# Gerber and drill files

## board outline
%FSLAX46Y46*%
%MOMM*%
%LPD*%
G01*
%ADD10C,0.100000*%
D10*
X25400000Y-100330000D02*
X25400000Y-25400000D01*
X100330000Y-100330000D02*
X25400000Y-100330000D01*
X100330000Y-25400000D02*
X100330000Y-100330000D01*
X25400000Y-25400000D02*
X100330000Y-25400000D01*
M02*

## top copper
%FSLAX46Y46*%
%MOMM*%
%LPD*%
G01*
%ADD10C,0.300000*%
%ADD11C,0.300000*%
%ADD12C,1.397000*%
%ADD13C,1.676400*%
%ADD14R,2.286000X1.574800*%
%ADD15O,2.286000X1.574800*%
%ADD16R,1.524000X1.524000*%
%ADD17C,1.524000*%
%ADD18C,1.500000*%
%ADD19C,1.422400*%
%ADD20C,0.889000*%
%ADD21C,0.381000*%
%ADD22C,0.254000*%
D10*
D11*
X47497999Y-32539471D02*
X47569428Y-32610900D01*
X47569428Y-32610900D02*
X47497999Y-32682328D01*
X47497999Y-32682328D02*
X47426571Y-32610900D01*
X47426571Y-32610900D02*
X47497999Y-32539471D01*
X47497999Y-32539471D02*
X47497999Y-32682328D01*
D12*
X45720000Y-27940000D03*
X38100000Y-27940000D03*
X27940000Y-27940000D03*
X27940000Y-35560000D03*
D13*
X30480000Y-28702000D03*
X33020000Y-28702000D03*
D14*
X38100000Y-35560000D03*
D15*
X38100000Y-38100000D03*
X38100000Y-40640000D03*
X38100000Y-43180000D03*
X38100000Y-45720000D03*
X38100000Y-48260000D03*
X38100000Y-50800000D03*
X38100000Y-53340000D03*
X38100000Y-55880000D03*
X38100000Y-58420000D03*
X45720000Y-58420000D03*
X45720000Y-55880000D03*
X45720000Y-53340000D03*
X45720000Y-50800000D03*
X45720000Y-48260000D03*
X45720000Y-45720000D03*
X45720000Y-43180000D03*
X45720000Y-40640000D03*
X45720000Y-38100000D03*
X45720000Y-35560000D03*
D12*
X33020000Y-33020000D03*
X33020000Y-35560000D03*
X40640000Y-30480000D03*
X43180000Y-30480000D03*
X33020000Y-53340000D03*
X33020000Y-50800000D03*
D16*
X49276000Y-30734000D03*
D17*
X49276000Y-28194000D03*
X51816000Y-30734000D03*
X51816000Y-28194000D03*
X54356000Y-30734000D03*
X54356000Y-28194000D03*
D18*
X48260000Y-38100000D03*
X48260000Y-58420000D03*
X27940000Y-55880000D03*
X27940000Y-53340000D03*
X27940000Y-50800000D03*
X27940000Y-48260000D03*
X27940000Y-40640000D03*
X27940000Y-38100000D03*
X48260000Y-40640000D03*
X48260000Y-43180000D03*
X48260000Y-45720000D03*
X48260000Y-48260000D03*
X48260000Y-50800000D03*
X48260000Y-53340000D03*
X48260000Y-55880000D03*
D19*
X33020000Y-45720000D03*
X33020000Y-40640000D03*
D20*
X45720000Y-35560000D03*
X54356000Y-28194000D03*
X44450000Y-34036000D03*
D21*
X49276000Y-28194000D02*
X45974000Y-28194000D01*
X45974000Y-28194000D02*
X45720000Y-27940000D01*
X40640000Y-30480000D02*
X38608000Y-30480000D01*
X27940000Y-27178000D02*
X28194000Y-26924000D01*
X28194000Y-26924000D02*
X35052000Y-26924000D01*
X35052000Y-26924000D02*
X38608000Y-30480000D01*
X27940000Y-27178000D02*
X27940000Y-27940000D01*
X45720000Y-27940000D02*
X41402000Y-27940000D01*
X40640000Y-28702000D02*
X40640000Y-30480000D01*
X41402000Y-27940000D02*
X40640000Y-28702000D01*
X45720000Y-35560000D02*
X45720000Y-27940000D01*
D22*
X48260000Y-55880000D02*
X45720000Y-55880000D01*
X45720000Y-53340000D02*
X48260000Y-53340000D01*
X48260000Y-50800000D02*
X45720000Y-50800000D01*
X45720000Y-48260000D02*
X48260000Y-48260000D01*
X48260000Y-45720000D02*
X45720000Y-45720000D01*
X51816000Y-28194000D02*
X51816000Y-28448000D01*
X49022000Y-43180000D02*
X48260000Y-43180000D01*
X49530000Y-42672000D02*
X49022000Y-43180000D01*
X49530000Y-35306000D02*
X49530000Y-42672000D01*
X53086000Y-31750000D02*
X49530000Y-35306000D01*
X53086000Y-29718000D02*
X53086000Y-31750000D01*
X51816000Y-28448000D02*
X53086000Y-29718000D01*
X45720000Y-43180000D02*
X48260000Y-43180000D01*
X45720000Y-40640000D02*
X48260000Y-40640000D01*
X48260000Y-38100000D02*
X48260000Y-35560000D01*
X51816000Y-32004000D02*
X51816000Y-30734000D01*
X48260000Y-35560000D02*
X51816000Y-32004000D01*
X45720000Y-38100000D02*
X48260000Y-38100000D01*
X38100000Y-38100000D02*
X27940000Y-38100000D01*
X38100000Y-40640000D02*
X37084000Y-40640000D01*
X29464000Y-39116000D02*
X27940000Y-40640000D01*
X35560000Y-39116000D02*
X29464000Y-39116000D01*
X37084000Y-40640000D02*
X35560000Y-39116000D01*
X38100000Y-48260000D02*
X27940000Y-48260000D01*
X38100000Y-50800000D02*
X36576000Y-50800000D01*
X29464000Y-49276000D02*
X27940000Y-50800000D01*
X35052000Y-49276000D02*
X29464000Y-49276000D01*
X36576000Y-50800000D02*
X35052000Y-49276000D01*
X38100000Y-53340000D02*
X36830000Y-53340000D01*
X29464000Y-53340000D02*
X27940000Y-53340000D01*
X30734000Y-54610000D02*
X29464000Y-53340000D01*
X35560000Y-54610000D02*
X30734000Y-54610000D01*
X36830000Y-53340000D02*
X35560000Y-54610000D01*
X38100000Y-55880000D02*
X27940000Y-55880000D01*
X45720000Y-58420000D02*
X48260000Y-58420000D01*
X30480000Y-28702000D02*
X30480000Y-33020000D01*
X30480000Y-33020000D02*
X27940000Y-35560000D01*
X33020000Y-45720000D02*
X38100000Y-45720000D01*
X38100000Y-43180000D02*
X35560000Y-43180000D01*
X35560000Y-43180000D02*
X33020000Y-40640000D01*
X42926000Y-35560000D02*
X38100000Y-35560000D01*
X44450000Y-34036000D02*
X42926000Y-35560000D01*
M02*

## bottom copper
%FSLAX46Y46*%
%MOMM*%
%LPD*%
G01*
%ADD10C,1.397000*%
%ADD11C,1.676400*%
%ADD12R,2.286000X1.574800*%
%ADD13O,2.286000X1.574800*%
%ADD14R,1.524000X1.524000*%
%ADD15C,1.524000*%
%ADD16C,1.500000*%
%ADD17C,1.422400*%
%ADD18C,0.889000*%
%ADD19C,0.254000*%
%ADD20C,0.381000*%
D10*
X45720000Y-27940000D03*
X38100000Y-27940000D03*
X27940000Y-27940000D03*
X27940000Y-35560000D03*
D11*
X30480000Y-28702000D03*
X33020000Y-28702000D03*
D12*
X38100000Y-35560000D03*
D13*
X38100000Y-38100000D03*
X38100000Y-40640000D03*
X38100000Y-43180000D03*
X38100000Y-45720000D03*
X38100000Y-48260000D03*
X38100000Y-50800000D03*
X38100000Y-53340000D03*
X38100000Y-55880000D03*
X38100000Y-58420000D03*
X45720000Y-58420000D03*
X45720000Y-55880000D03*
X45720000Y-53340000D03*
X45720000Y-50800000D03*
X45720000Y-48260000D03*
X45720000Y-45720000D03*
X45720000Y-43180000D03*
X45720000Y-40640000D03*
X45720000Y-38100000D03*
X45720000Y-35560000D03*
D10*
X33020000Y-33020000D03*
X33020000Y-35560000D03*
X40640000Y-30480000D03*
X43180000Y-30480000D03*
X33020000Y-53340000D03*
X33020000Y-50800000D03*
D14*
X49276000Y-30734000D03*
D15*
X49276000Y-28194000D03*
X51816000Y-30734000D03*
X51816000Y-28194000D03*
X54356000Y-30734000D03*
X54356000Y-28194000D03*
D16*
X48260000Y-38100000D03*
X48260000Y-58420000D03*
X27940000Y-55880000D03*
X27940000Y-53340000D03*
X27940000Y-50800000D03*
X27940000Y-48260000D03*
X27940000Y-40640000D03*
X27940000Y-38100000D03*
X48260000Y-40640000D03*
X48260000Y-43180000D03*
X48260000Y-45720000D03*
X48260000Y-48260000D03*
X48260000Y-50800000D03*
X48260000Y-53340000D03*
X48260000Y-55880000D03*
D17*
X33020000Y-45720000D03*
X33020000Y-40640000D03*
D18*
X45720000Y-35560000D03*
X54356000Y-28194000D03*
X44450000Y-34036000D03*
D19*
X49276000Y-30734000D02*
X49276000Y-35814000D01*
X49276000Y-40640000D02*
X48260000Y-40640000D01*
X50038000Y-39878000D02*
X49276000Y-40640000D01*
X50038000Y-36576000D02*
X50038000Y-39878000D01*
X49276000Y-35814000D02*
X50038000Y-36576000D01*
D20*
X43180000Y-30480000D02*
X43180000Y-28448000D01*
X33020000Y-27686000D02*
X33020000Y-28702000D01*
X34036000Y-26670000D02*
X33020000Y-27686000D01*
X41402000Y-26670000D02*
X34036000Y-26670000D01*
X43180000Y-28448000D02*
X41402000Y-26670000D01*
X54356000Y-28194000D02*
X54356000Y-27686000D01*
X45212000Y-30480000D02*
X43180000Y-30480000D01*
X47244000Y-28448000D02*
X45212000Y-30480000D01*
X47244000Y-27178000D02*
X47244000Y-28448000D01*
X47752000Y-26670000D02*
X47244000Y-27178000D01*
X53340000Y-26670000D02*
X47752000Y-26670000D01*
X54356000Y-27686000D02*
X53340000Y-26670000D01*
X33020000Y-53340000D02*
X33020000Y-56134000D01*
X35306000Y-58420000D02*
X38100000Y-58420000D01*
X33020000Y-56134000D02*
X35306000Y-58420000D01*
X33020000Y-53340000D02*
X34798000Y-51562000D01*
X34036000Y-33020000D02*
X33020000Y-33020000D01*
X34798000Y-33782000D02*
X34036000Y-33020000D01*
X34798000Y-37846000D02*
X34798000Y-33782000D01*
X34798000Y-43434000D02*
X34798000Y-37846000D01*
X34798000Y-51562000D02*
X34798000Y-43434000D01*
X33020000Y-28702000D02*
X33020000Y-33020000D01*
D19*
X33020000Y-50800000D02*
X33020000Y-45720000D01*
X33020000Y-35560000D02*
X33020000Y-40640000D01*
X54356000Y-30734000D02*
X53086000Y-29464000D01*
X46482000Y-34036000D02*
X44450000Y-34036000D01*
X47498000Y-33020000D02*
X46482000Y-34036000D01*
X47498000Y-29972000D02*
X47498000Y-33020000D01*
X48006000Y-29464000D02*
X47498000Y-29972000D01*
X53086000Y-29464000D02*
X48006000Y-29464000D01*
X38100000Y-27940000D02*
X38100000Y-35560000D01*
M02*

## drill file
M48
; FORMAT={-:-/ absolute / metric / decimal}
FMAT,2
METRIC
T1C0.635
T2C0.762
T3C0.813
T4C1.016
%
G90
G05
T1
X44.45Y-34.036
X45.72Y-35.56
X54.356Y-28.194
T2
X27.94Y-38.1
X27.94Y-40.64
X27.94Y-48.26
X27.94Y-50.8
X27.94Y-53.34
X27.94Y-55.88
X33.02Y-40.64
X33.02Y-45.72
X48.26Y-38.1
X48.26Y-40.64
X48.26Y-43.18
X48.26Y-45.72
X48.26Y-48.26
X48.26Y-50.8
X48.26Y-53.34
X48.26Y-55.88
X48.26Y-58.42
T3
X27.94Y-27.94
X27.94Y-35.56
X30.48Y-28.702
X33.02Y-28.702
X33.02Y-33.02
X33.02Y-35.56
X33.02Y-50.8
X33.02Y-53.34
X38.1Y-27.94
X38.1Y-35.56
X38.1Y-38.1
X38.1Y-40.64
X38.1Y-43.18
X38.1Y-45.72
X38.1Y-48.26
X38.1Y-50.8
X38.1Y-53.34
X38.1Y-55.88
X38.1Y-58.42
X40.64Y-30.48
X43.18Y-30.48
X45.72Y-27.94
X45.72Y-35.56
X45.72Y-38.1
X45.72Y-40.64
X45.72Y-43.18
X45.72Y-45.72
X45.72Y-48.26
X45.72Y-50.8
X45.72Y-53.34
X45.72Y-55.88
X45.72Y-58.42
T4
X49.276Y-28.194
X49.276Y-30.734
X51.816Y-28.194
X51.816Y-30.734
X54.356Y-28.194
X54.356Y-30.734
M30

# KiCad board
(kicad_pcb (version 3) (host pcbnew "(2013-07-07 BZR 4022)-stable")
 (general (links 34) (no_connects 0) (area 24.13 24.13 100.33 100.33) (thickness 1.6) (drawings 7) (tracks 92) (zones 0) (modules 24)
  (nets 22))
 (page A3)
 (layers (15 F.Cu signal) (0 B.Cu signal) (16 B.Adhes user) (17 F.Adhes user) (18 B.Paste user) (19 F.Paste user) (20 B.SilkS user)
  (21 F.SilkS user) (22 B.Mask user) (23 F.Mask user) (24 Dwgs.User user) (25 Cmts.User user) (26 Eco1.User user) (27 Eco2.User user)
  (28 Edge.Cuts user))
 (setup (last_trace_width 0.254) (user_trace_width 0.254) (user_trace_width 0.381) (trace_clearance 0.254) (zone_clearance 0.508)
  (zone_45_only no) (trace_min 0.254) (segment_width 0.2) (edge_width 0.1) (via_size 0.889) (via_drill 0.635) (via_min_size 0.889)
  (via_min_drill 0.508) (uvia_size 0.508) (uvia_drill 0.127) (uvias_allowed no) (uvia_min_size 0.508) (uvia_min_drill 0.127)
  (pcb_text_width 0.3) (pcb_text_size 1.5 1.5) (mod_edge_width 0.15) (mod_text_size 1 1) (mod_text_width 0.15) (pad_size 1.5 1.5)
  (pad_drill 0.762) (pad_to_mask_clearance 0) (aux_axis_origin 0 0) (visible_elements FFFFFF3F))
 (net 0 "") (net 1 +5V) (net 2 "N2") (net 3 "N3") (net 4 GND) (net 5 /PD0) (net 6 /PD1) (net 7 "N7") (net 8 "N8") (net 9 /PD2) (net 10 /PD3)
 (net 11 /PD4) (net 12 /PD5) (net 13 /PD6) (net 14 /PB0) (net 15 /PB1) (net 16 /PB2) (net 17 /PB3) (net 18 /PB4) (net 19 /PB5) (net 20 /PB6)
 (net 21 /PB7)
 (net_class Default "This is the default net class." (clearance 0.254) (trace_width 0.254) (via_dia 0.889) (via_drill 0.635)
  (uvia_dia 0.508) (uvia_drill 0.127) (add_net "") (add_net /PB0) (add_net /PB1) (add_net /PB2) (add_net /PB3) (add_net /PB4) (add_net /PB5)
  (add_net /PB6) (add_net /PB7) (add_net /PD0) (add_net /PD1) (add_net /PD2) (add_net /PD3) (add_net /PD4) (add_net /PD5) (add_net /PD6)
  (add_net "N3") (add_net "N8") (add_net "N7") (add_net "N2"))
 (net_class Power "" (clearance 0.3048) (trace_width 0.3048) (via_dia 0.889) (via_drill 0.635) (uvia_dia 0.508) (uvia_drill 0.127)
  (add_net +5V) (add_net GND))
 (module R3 (layer F.Cu) (at 41.91 27.94 180) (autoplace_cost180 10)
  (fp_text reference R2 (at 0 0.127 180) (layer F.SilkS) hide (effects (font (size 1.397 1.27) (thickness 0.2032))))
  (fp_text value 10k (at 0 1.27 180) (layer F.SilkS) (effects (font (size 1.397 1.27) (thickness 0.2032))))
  (pad 1 thru_hole circle (at -3.81 0 180) (size 1.397 1.397) (drill 0.8128) (layers *.Cu *.Mask F.SilkS) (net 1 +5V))
  (pad 2 thru_hole circle (at 3.81 0 180) (size 1.397 1.397) (drill 0.8128) (layers *.Cu *.Mask F.SilkS) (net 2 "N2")))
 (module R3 (layer F.Cu) (at 27.94 31.75 270) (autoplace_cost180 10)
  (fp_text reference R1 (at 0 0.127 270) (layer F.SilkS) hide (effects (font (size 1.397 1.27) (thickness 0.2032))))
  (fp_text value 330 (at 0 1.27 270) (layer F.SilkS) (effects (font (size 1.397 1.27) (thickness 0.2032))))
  (pad 1 thru_hole circle (at -3.81 0 270) (size 1.397 1.397) (drill 0.8128) (layers *.Cu *.Mask F.SilkS) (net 1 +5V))
  (pad 2 thru_hole circle (at 3.81 0 270) (size 1.397 1.397) (drill 0.8128) (layers *.Cu *.Mask F.SilkS) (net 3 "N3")))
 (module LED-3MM (layer F.Cu) (at 31.75 28.702)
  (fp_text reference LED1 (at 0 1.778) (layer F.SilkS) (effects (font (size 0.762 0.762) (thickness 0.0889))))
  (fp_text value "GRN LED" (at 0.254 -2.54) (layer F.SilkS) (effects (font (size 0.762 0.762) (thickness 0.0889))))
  (pad 1 thru_hole circle (at -1.27 0) (size 1.6764 1.6764) (drill 0.8128) (layers *.Cu *.Mask F.SilkS) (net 3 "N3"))
  (pad 2 thru_hole circle (at 1.27 0) (size 1.6764 1.6764) (drill 0.8128) (layers *.Cu *.Mask F.SilkS) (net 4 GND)))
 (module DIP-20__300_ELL (layer F.Cu) (at 41.91 46.99 270)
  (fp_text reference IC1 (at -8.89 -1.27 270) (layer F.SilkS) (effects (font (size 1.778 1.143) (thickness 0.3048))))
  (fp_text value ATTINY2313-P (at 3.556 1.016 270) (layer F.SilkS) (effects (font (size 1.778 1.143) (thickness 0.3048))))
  (pad 1 thru_hole rect (at -11.43 3.81 270) (size 1.5748 2.286) (drill 0.8128) (layers *.Cu *.Mask F.SilkS) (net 2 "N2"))
  (pad 2 thru_hole oval (at -8.89 3.81 270) (size 1.5748 2.286) (drill 0.8128) (layers *.Cu *.Mask F.SilkS) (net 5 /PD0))
  (pad 3 thru_hole oval (at -6.35 3.81 270) (size 1.5748 2.286) (drill 0.8128) (layers *.Cu *.Mask F.SilkS) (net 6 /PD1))
  (pad 4 thru_hole oval (at -3.81 3.81 270) (size 1.5748 2.286) (drill 0.8128) (layers *.Cu *.Mask F.SilkS) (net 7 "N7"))
  (pad 5 thru_hole oval (at -1.27 3.81 270) (size 1.5748 2.286) (drill 0.8128) (layers *.Cu *.Mask F.SilkS) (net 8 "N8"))
  (pad 6 thru_hole oval (at 1.27 3.81 270) (size 1.5748 2.286) (drill 0.8128) (layers *.Cu *.Mask F.SilkS) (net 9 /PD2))
  (pad 7 thru_hole oval (at 3.81 3.81 270) (size 1.5748 2.286) (drill 0.8128) (layers *.Cu *.Mask F.SilkS) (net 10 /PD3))
  (pad 8 thru_hole oval (at 6.35 3.81 270) (size 1.5748 2.286) (drill 0.8128) (layers *.Cu *.Mask F.SilkS) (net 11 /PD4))
  (pad 9 thru_hole oval (at 8.89 3.81 270) (size 1.5748 2.286) (drill 0.8128) (layers *.Cu *.Mask F.SilkS) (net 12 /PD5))
  (pad 10 thru_hole oval (at 11.43 3.81 270) (size 1.5748 2.286) (drill 0.8128) (layers *.Cu *.Mask F.SilkS) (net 4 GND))
  (pad 11 thru_hole oval (at 11.43 -3.81 270) (size 1.5748 2.286) (drill 0.8128) (layers *.Cu *.Mask F.SilkS) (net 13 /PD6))
  (pad 12 thru_hole oval (at 8.89 -3.81 270) (size 1.5748 2.286) (drill 0.8128) (layers *.Cu *.Mask F.SilkS) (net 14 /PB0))
  (pad 13 thru_hole oval (at 6.35 -3.81 270) (size 1.5748 2.286) (drill 0.8128) (layers *.Cu *.Mask F.SilkS) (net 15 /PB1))
  (pad 14 thru_hole oval (at 3.81 -3.81 270) (size 1.5748 2.286) (drill 0.8128) (layers *.Cu *.Mask F.SilkS) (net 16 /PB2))
  (pad 15 thru_hole oval (at 1.27 -3.81 270) (size 1.5748 2.286) (drill 0.8128) (layers *.Cu *.Mask F.SilkS) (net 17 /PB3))
  (pad 16 thru_hole oval (at -1.27 -3.81 270) (size 1.5748 2.286) (drill 0.8128) (layers *.Cu *.Mask F.SilkS) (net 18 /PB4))
  (pad 17 thru_hole oval (at -3.81 -3.81 270) (size 1.5748 2.286) (drill 0.8128) (layers *.Cu *.Mask F.SilkS) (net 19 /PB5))
  (pad 18 thru_hole oval (at -6.35 -3.81 270) (size 1.5748 2.286) (drill 0.8128) (layers *.Cu *.Mask F.SilkS) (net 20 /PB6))
  (pad 19 thru_hole oval (at -8.89 -3.81 270) (size 1.5748 2.286) (drill 0.8128) (layers *.Cu *.Mask F.SilkS) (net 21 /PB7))
  (pad 20 thru_hole oval (at -11.43 -3.81 270) (size 1.5748 2.286) (drill 0.8128) (layers *.Cu *.Mask F.SilkS) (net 1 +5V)))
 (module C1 (layer F.Cu) (at 33.02 34.29 270)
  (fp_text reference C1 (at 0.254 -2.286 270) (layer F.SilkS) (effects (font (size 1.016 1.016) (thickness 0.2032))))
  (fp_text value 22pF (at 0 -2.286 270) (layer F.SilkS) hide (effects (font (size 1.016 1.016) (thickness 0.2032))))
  (pad 1 thru_hole circle (at -1.27 0 270) (size 1.397 1.397) (drill 0.8128) (layers *.Cu *.Mask F.SilkS) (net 4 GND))
  (pad 2 thru_hole circle (at 1.27 0 270) (size 1.397 1.397) (drill 0.8128) (layers *.Cu *.Mask F.SilkS) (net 7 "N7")))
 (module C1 (layer F.Cu) (at 41.91 30.48)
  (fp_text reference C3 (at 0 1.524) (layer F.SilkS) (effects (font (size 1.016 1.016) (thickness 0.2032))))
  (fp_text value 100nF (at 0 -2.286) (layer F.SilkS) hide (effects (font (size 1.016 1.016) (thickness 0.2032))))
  (pad 1 thru_hole circle (at -1.27 0) (size 1.397 1.397) (drill 0.8128) (layers *.Cu *.Mask F.SilkS) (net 1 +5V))
  (pad 2 thru_hole circle (at 1.27 0) (size 1.397 1.397) (drill 0.8128) (layers *.Cu *.Mask F.SilkS) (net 4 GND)))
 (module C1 (layer F.Cu) (at 33.02 52.07 90)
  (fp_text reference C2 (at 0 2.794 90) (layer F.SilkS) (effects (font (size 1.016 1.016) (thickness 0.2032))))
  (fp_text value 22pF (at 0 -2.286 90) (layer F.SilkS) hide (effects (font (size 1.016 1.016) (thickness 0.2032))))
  (pad 1 thru_hole circle (at -1.27 0 90) (size 1.397 1.397) (drill 0.8128) (layers *.Cu *.Mask F.SilkS) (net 4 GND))
  (pad 2 thru_hole circle (at 1.27 0 90) (size 1.397 1.397) (drill 0.8128) (layers *.Cu *.Mask F.SilkS) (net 8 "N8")))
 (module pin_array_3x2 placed (layer F.Cu) (at 51.816 29.464)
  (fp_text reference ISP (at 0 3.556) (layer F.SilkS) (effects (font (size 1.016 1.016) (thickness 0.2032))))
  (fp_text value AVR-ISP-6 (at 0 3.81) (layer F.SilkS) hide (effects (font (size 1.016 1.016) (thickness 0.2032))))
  (pad 1 thru_hole rect (at -2.54 1.27) (size 1.524 1.524) (drill 1.016) (layers *.Cu *.Mask F.SilkS) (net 20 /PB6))
  (pad 2 thru_hole circle (at -2.54 -1.27) (size 1.524 1.524) (drill 1.016) (layers *.Cu *.Mask F.SilkS) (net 1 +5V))
  (pad 3 thru_hole circle (at 0 1.27) (size 1.524 1.524) (drill 1.016) (layers *.Cu *.Mask F.SilkS) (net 21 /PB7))
  (pad 4 thru_hole circle (at 0 -1.27) (size 1.524 1.524) (drill 1.016) (layers *.Cu *.Mask F.SilkS) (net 19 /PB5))
  (pad 5 thru_hole circle (at 2.54 1.27) (size 1.524 1.524) (drill 1.016) (layers *.Cu *.Mask F.SilkS) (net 2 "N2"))
  (pad 6 thru_hole circle (at 2.54 -1.27) (size 1.524 1.524) (drill 1.016) (layers *.Cu *.Mask F.SilkS) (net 4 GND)))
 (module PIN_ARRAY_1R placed (layer F.Cu) (at 48.26 38.1)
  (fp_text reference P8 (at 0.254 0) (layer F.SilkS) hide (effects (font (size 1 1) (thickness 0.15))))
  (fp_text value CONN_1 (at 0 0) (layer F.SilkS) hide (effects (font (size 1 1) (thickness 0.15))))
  (pad 1 thru_hole circle (at 0 0) (size 1.5 1.5) (drill 0.762) (layers *.Cu *.Mask F.SilkS) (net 21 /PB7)))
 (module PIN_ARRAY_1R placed (layer F.Cu) (at 48.26 58.42)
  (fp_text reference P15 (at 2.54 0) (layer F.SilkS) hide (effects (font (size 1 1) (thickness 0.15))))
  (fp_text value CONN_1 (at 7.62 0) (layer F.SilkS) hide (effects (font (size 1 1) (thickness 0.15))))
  (pad 1 thru_hole circle (at 0 0) (size 1.5 1.5) (drill 0.762) (layers *.Cu *.Mask F.SilkS) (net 13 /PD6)))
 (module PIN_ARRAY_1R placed (layer F.Cu) (at 27.94 55.88)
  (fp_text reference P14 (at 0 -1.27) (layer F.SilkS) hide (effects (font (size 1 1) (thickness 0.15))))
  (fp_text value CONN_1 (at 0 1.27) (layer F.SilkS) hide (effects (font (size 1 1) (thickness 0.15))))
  (pad 1 thru_hole circle (at 0 0) (size 1.5 1.5) (drill 0.762) (layers *.Cu *.Mask F.SilkS) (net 12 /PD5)))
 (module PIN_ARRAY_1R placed (layer F.Cu) (at 27.94 53.34)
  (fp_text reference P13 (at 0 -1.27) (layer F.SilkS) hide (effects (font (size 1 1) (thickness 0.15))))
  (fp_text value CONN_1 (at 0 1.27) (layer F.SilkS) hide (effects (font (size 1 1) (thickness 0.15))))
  (pad 1 thru_hole circle (at 0 0) (size 1.5 1.5) (drill 0.762) (layers *.Cu *.Mask F.SilkS) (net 11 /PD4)))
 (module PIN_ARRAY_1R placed (layer F.Cu) (at 27.94 50.8)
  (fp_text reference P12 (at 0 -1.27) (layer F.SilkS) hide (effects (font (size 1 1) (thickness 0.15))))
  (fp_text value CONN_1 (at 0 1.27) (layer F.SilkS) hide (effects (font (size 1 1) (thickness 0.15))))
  (pad 1 thru_hole circle (at 0 0) (size 1.5 1.5) (drill 0.762) (layers *.Cu *.Mask F.SilkS) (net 10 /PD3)))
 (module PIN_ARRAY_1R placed (layer F.Cu) (at 27.94 48.26)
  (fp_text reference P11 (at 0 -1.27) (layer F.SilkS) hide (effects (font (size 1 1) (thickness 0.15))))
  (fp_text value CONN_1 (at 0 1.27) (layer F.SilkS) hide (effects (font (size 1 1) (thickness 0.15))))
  (pad 1 thru_hole circle (at 0 0) (size 1.5 1.5) (drill 0.762) (layers *.Cu *.Mask F.SilkS) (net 9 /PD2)))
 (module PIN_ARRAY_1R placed (layer F.Cu) (at 27.94 40.64)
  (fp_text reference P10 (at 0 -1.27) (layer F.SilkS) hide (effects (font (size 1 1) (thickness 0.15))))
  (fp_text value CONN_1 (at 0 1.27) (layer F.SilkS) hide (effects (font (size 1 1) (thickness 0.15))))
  (pad 1 thru_hole circle (at 0 0) (size 1.5 1.5) (drill 0.762) (layers *.Cu *.Mask F.SilkS) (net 6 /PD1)))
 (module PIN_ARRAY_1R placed (layer F.Cu) (at 27.94 38.1)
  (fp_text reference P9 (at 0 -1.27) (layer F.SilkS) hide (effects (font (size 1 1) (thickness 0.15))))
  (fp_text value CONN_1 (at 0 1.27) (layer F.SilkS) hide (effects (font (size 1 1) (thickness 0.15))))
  (pad 1 thru_hole circle (at 0 0) (size 1.5 1.5) (drill 0.762) (layers *.Cu *.Mask F.SilkS) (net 5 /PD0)))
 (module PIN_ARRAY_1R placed (layer F.Cu) (at 48.26 40.64)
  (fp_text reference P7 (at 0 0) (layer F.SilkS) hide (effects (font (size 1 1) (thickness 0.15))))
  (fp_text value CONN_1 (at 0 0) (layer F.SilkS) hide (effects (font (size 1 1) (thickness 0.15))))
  (pad 1 thru_hole circle (at 0 0) (size 1.5 1.5) (drill 0.762) (layers *.Cu *.Mask F.SilkS) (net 20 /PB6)))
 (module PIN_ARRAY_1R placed (layer F.Cu) (at 48.26 43.18)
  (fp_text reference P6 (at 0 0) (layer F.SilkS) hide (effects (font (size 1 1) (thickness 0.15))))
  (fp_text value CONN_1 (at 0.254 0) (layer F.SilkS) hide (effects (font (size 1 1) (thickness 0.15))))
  (pad 1 thru_hole circle (at 0 0) (size 1.5 1.5) (drill 0.762) (layers *.Cu *.Mask F.SilkS) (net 19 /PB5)))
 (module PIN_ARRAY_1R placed (layer F.Cu) (at 48.26 45.72)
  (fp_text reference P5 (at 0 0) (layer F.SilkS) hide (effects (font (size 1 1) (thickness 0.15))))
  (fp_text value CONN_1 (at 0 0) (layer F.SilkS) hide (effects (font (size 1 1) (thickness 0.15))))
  (pad 1 thru_hole circle (at 0 0) (size 1.5 1.5) (drill 0.762) (layers *.Cu *.Mask F.SilkS) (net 18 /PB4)))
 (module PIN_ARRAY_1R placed (layer F.Cu) (at 48.26 48.26)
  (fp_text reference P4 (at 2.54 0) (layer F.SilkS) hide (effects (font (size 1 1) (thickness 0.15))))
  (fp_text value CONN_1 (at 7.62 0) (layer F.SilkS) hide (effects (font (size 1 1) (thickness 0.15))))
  (pad 1 thru_hole circle (at 0 0) (size 1.5 1.5) (drill 0.762) (layers *.Cu *.Mask F.SilkS) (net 17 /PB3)))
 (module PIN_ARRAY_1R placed (layer F.Cu) (at 48.26 50.8)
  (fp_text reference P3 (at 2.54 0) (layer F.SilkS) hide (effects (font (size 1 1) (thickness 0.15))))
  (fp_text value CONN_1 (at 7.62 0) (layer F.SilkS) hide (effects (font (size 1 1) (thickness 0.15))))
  (pad 1 thru_hole circle (at 0 0) (size 1.5 1.5) (drill 0.762) (layers *.Cu *.Mask F.SilkS) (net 16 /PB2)))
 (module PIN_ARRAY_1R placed (layer F.Cu) (at 48.26 53.34)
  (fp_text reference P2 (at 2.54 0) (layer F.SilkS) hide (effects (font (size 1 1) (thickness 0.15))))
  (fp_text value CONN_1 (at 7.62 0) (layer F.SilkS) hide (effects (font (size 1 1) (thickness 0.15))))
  (pad 1 thru_hole circle (at 0 0) (size 1.5 1.5) (drill 0.762) (layers *.Cu *.Mask F.SilkS) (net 15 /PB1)))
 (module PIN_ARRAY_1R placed (layer F.Cu) (at 48.26 55.88)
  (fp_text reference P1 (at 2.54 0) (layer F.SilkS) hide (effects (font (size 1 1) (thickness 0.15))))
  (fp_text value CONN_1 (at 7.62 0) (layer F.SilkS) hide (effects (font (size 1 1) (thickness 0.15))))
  (pad 1 thru_hole circle (at 0 0) (size 1.5 1.5) (drill 0.762) (layers *.Cu *.Mask F.SilkS) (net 14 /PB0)))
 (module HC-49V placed (layer F.Cu) (at 33.02 43.18 90) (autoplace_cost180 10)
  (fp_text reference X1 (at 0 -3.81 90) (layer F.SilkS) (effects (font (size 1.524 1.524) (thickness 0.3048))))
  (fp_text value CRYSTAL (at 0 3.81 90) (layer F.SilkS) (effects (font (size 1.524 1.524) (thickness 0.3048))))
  (pad 1 thru_hole circle (at -2.54 0 90) (size 1.4224 1.4224) (drill 0.762) (layers *.Cu *.Mask F.SilkS) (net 8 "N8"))
  (pad 2 thru_hole circle (at 2.54 0 90) (size 1.4224 1.4224) (drill 0.762) (layers *.Cu *.Mask F.SilkS) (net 7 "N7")))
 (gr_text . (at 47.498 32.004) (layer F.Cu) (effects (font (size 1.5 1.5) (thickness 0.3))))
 (gr_line (start 25.4 100.33) (end 25.4 25.4) (angle 90) (layer Edge.Cuts) (width 0.1))
 (gr_line (start 100.33 100.33) (end 25.4 100.33) (angle 90) (layer Edge.Cuts) (width 0.1))
 (gr_line (start 100.33 25.4) (end 100.33 100.33) (angle 90) (layer Edge.Cuts) (width 0.1))
 (gr_line (start 25.4 25.4) (end 100.33 25.4) (angle 90) (layer Edge.Cuts) (width 0.1))
 (segment (start 49.276 28.194) (end 45.974 28.194) (width 0.381) (layer F.Cu) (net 1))
 (segment (start 45.974 28.194) (end 45.72 27.94) (width 0.381) (layer F.Cu) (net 1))
 (segment (start 40.64 30.48) (end 38.608 30.48) (width 0.381) (layer F.Cu) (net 1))
 (segment (start 27.94 27.178) (end 28.194 26.924) (width 0.381) (layer F.Cu) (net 1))
 (segment (start 28.194 26.924) (end 35.052 26.924) (width 0.381) (layer F.Cu) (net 1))
 (segment (start 35.052 26.924) (end 38.608 30.48) (width 0.381) (layer F.Cu) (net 1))
 (segment (start 27.94 27.178) (end 27.94 27.94) (width 0.381) (layer F.Cu) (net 1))
 (segment (start 45.72 27.94) (end 41.402 27.94) (width 0.381) (layer F.Cu) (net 1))
 (segment (start 40.64 28.702) (end 40.64 30.48) (width 0.381) (layer F.Cu) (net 1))
 (segment (start 41.402 27.94) (end 40.64 28.702) (width 0.381) (layer F.Cu) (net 1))
 (via (at 45.72 35.56) (size 0.889) (layers F.Cu B.Cu) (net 1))
 (segment (start 45.72 35.56) (end 45.72 27.94) (width 0.381) (layer F.Cu) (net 1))
 (segment (start 48.26 55.88) (end 45.72 55.88) (width 0.254) (layer F.Cu) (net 14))
 (segment (start 45.72 53.34) (end 48.26 53.34) (width 0.254) (layer F.Cu) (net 15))
 (segment (start 48.26 50.8) (end 45.72 50.8) (width 0.254) (layer F.Cu) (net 16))
 (segment (start 45.72 48.26) (end 48.26 48.26) (width 0.254) (layer F.Cu) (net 17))
 (segment (start 48.26 45.72) (end 45.72 45.72) (width 0.254) (layer F.Cu) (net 18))
 (segment (start 51.816 28.194) (end 51.816 28.448) (width 0.254) (layer F.Cu) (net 19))
 (segment (start 49.022 43.18) (end 48.26 43.18) (width 0.254) (layer F.Cu) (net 19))
 (segment (start 49.53 42.672) (end 49.022 43.18) (width 0.254) (layer F.Cu) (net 19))
 (segment (start 49.53 35.306) (end 49.53 42.672) (width 0.254) (layer F.Cu) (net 19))
 (segment (start 53.086 31.75) (end 49.53 35.306) (width 0.254) (layer F.Cu) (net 19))
 (segment (start 53.086 29.718) (end 53.086 31.75) (width 0.254) (layer F.Cu) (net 19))
 (segment (start 51.816 28.448) (end 53.086 29.718) (width 0.254) (layer F.Cu) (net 19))
 (segment (start 45.72 43.18) (end 48.26 43.18) (width 0.254) (layer F.Cu) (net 19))
 (segment (start 49.276 30.734) (end 49.276 35.814) (width 0.254) (layer B.Cu) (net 20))
 (segment (start 49.276 40.64) (end 48.26 40.64) (width 0.254) (layer B.Cu) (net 20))
 (segment (start 50.038 39.878) (end 49.276 40.64) (width 0.254) (layer B.Cu) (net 20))
 (segment (start 50.038 36.576) (end 50.038 39.878) (width 0.254) (layer B.Cu) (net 20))
 (segment (start 49.276 35.814) (end 50.038 36.576) (width 0.254) (layer B.Cu) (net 20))
 (segment (start 45.72 40.64) (end 48.26 40.64) (width 0.254) (layer F.Cu) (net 20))
 (segment (start 48.26 38.1) (end 48.26 35.56) (width 0.254) (layer F.Cu) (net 21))
 (segment (start 51.816 32.004) (end 51.816 30.734) (width 0.254) (layer F.Cu) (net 21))
 (segment (start 48.26 35.56) (end 51.816 32.004) (width 0.254) (layer F.Cu) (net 21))
 (segment (start 45.72 38.1) (end 48.26 38.1) (width 0.254) (layer F.Cu) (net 21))
 (segment (start 38.1 38.1) (end 27.94 38.1) (width 0.254) (layer F.Cu) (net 5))
 (segment (start 38.1 40.64) (end 37.084 40.64) (width 0.254) (layer F.Cu) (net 6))
 (segment (start 29.464 39.116) (end 27.94 40.64) (width 0.254) (layer F.Cu) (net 6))
 (segment (start 35.56 39.116) (end 29.464 39.116) (width 0.254) (layer F.Cu) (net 6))
 (segment (start 37.084 40.64) (end 35.56 39.116) (width 0.254) (layer F.Cu) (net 6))
 (segment (start 38.1 48.26) (end 27.94 48.26) (width 0.254) (layer F.Cu) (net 9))
 (segment (start 38.1 50.8) (end 36.576 50.8) (width 0.254) (layer F.Cu) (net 10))
 (segment (start 29.464 49.276) (end 27.94 50.8) (width 0.254) (layer F.Cu) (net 10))
 (segment (start 35.052 49.276) (end 29.464 49.276) (width 0.254) (layer F.Cu) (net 10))
 (segment (start 36.576 50.8) (end 35.052 49.276) (width 0.254) (layer F.Cu) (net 10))
 (segment (start 38.1 53.34) (end 36.83 53.34) (width 0.254) (layer F.Cu) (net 11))
 (segment (start 29.464 53.34) (end 27.94 53.34) (width 0.254) (layer F.Cu) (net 11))
 (segment (start 30.734 54.61) (end 29.464 53.34) (width 0.254) (layer F.Cu) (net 11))
 (segment (start 35.56 54.61) (end 30.734 54.61) (width 0.254) (layer F.Cu) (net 11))
 (segment (start 36.83 53.34) (end 35.56 54.61) (width 0.254) (layer F.Cu) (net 11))
 (segment (start 38.1 55.88) (end 27.94 55.88) (width 0.254) (layer F.Cu) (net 12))
 (segment (start 45.72 58.42) (end 48.26 58.42) (width 0.254) (layer F.Cu) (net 13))
 (segment (start 43.18 30.48) (end 43.18 28.448) (width 0.381) (layer B.Cu) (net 4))
 (segment (start 33.02 27.686) (end 33.02 28.702) (width 0.381) (layer B.Cu) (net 4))
 (segment (start 34.036 26.67) (end 33.02 27.686) (width 0.381) (layer B.Cu) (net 4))
 (segment (start 41.402 26.67) (end 34.036 26.67) (width 0.381) (layer B.Cu) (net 4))
 (segment (start 43.18 28.448) (end 41.402 26.67) (width 0.381) (layer B.Cu) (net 4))
 (segment (start 54.356 28.194) (end 54.356 27.686) (width 0.381) (layer B.Cu) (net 4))
 (segment (start 45.212 30.48) (end 43.18 30.48) (width 0.381) (layer B.Cu) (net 4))
 (segment (start 47.244 28.448) (end 45.212 30.48) (width 0.381) (layer B.Cu) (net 4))
 (segment (start 47.244 27.178) (end 47.244 28.448) (width 0.381) (layer B.Cu) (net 4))
 (segment (start 47.752 26.67) (end 47.244 27.178) (width 0.381) (layer B.Cu) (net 4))
 (segment (start 53.34 26.67) (end 47.752 26.67) (width 0.381) (layer B.Cu) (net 4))
 (segment (start 54.356 27.686) (end 53.34 26.67) (width 0.381) (layer B.Cu) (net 4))
 (segment (start 33.02 53.34) (end 33.02 56.134) (width 0.381) (layer B.Cu) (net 4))
 (segment (start 35.306 58.42) (end 38.1 58.42) (width 0.381) (layer B.Cu) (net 4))
 (segment (start 33.02 56.134) (end 35.306 58.42) (width 0.381) (layer B.Cu) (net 4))
 (segment (start 33.02 53.34) (end 34.798 51.562) (width 0.381) (layer B.Cu) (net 4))
 (segment (start 34.036 33.02) (end 33.02 33.02) (width 0.381) (layer B.Cu) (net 4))
 (segment (start 34.798 33.782) (end 34.036 33.02) (width 0.381) (layer B.Cu) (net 4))
 (segment (start 34.798 37.846) (end 34.798 33.782) (width 0.381) (layer B.Cu) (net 4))
 (segment (start 34.798 43.434) (end 34.798 37.846) (width 0.381) (layer B.Cu) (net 4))
 (segment (start 34.798 51.562) (end 34.798 43.434) (width 0.381) (layer B.Cu) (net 4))
 (segment (start 33.02 28.702) (end 33.02 33.02) (width 0.381) (layer B.Cu) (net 4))
 (via (at 54.356 28.194) (size 0.889) (layers F.Cu B.Cu) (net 4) (status 30))
 (segment (start 30.48 28.702) (end 30.48 33.02) (width 0.254) (layer F.Cu) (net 3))
 (segment (start 30.48 33.02) (end 27.94 35.56) (width 0.254) (layer F.Cu) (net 3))
 (segment (start 33.02 45.72) (end 38.1 45.72) (width 0.254) (layer F.Cu) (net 8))
 (segment (start 33.02 50.8) (end 33.02 45.72) (width 0.254) (layer B.Cu) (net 8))
 (segment (start 38.1 43.18) (end 35.56 43.18) (width 0.254) (layer F.Cu) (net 7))
 (segment (start 35.56 43.18) (end 33.02 40.64) (width 0.254) (layer F.Cu) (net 7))
 (segment (start 33.02 35.56) (end 33.02 40.64) (width 0.254) (layer B.Cu) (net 7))
 (segment (start 54.356 30.734) (end 53.086 29.464) (width 0.254) (layer B.Cu) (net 2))
 (segment (start 42.926 35.56) (end 38.1 35.56) (width 0.254) (layer F.Cu) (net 2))
 (segment (start 44.45 34.036) (end 42.926 35.56) (width 0.254) (layer F.Cu) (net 2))
 (via (at 44.45 34.036) (size 0.889) (layers F.Cu B.Cu) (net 2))
 (segment (start 46.482 34.036) (end 44.45 34.036) (width 0.254) (layer B.Cu) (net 2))
 (segment (start 47.498 33.02) (end 46.482 34.036) (width 0.254) (layer B.Cu) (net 2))
 (segment (start 47.498 29.972) (end 47.498 33.02) (width 0.254) (layer B.Cu) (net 2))
 (segment (start 48.006 29.464) (end 47.498 29.972) (width 0.254) (layer B.Cu) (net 2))
 (segment (start 53.086 29.464) (end 48.006 29.464) (width 0.254) (layer B.Cu) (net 2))
 (segment (start 38.1 27.94) (end 38.1 35.56) (width 0.254) (layer B.Cu) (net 2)))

